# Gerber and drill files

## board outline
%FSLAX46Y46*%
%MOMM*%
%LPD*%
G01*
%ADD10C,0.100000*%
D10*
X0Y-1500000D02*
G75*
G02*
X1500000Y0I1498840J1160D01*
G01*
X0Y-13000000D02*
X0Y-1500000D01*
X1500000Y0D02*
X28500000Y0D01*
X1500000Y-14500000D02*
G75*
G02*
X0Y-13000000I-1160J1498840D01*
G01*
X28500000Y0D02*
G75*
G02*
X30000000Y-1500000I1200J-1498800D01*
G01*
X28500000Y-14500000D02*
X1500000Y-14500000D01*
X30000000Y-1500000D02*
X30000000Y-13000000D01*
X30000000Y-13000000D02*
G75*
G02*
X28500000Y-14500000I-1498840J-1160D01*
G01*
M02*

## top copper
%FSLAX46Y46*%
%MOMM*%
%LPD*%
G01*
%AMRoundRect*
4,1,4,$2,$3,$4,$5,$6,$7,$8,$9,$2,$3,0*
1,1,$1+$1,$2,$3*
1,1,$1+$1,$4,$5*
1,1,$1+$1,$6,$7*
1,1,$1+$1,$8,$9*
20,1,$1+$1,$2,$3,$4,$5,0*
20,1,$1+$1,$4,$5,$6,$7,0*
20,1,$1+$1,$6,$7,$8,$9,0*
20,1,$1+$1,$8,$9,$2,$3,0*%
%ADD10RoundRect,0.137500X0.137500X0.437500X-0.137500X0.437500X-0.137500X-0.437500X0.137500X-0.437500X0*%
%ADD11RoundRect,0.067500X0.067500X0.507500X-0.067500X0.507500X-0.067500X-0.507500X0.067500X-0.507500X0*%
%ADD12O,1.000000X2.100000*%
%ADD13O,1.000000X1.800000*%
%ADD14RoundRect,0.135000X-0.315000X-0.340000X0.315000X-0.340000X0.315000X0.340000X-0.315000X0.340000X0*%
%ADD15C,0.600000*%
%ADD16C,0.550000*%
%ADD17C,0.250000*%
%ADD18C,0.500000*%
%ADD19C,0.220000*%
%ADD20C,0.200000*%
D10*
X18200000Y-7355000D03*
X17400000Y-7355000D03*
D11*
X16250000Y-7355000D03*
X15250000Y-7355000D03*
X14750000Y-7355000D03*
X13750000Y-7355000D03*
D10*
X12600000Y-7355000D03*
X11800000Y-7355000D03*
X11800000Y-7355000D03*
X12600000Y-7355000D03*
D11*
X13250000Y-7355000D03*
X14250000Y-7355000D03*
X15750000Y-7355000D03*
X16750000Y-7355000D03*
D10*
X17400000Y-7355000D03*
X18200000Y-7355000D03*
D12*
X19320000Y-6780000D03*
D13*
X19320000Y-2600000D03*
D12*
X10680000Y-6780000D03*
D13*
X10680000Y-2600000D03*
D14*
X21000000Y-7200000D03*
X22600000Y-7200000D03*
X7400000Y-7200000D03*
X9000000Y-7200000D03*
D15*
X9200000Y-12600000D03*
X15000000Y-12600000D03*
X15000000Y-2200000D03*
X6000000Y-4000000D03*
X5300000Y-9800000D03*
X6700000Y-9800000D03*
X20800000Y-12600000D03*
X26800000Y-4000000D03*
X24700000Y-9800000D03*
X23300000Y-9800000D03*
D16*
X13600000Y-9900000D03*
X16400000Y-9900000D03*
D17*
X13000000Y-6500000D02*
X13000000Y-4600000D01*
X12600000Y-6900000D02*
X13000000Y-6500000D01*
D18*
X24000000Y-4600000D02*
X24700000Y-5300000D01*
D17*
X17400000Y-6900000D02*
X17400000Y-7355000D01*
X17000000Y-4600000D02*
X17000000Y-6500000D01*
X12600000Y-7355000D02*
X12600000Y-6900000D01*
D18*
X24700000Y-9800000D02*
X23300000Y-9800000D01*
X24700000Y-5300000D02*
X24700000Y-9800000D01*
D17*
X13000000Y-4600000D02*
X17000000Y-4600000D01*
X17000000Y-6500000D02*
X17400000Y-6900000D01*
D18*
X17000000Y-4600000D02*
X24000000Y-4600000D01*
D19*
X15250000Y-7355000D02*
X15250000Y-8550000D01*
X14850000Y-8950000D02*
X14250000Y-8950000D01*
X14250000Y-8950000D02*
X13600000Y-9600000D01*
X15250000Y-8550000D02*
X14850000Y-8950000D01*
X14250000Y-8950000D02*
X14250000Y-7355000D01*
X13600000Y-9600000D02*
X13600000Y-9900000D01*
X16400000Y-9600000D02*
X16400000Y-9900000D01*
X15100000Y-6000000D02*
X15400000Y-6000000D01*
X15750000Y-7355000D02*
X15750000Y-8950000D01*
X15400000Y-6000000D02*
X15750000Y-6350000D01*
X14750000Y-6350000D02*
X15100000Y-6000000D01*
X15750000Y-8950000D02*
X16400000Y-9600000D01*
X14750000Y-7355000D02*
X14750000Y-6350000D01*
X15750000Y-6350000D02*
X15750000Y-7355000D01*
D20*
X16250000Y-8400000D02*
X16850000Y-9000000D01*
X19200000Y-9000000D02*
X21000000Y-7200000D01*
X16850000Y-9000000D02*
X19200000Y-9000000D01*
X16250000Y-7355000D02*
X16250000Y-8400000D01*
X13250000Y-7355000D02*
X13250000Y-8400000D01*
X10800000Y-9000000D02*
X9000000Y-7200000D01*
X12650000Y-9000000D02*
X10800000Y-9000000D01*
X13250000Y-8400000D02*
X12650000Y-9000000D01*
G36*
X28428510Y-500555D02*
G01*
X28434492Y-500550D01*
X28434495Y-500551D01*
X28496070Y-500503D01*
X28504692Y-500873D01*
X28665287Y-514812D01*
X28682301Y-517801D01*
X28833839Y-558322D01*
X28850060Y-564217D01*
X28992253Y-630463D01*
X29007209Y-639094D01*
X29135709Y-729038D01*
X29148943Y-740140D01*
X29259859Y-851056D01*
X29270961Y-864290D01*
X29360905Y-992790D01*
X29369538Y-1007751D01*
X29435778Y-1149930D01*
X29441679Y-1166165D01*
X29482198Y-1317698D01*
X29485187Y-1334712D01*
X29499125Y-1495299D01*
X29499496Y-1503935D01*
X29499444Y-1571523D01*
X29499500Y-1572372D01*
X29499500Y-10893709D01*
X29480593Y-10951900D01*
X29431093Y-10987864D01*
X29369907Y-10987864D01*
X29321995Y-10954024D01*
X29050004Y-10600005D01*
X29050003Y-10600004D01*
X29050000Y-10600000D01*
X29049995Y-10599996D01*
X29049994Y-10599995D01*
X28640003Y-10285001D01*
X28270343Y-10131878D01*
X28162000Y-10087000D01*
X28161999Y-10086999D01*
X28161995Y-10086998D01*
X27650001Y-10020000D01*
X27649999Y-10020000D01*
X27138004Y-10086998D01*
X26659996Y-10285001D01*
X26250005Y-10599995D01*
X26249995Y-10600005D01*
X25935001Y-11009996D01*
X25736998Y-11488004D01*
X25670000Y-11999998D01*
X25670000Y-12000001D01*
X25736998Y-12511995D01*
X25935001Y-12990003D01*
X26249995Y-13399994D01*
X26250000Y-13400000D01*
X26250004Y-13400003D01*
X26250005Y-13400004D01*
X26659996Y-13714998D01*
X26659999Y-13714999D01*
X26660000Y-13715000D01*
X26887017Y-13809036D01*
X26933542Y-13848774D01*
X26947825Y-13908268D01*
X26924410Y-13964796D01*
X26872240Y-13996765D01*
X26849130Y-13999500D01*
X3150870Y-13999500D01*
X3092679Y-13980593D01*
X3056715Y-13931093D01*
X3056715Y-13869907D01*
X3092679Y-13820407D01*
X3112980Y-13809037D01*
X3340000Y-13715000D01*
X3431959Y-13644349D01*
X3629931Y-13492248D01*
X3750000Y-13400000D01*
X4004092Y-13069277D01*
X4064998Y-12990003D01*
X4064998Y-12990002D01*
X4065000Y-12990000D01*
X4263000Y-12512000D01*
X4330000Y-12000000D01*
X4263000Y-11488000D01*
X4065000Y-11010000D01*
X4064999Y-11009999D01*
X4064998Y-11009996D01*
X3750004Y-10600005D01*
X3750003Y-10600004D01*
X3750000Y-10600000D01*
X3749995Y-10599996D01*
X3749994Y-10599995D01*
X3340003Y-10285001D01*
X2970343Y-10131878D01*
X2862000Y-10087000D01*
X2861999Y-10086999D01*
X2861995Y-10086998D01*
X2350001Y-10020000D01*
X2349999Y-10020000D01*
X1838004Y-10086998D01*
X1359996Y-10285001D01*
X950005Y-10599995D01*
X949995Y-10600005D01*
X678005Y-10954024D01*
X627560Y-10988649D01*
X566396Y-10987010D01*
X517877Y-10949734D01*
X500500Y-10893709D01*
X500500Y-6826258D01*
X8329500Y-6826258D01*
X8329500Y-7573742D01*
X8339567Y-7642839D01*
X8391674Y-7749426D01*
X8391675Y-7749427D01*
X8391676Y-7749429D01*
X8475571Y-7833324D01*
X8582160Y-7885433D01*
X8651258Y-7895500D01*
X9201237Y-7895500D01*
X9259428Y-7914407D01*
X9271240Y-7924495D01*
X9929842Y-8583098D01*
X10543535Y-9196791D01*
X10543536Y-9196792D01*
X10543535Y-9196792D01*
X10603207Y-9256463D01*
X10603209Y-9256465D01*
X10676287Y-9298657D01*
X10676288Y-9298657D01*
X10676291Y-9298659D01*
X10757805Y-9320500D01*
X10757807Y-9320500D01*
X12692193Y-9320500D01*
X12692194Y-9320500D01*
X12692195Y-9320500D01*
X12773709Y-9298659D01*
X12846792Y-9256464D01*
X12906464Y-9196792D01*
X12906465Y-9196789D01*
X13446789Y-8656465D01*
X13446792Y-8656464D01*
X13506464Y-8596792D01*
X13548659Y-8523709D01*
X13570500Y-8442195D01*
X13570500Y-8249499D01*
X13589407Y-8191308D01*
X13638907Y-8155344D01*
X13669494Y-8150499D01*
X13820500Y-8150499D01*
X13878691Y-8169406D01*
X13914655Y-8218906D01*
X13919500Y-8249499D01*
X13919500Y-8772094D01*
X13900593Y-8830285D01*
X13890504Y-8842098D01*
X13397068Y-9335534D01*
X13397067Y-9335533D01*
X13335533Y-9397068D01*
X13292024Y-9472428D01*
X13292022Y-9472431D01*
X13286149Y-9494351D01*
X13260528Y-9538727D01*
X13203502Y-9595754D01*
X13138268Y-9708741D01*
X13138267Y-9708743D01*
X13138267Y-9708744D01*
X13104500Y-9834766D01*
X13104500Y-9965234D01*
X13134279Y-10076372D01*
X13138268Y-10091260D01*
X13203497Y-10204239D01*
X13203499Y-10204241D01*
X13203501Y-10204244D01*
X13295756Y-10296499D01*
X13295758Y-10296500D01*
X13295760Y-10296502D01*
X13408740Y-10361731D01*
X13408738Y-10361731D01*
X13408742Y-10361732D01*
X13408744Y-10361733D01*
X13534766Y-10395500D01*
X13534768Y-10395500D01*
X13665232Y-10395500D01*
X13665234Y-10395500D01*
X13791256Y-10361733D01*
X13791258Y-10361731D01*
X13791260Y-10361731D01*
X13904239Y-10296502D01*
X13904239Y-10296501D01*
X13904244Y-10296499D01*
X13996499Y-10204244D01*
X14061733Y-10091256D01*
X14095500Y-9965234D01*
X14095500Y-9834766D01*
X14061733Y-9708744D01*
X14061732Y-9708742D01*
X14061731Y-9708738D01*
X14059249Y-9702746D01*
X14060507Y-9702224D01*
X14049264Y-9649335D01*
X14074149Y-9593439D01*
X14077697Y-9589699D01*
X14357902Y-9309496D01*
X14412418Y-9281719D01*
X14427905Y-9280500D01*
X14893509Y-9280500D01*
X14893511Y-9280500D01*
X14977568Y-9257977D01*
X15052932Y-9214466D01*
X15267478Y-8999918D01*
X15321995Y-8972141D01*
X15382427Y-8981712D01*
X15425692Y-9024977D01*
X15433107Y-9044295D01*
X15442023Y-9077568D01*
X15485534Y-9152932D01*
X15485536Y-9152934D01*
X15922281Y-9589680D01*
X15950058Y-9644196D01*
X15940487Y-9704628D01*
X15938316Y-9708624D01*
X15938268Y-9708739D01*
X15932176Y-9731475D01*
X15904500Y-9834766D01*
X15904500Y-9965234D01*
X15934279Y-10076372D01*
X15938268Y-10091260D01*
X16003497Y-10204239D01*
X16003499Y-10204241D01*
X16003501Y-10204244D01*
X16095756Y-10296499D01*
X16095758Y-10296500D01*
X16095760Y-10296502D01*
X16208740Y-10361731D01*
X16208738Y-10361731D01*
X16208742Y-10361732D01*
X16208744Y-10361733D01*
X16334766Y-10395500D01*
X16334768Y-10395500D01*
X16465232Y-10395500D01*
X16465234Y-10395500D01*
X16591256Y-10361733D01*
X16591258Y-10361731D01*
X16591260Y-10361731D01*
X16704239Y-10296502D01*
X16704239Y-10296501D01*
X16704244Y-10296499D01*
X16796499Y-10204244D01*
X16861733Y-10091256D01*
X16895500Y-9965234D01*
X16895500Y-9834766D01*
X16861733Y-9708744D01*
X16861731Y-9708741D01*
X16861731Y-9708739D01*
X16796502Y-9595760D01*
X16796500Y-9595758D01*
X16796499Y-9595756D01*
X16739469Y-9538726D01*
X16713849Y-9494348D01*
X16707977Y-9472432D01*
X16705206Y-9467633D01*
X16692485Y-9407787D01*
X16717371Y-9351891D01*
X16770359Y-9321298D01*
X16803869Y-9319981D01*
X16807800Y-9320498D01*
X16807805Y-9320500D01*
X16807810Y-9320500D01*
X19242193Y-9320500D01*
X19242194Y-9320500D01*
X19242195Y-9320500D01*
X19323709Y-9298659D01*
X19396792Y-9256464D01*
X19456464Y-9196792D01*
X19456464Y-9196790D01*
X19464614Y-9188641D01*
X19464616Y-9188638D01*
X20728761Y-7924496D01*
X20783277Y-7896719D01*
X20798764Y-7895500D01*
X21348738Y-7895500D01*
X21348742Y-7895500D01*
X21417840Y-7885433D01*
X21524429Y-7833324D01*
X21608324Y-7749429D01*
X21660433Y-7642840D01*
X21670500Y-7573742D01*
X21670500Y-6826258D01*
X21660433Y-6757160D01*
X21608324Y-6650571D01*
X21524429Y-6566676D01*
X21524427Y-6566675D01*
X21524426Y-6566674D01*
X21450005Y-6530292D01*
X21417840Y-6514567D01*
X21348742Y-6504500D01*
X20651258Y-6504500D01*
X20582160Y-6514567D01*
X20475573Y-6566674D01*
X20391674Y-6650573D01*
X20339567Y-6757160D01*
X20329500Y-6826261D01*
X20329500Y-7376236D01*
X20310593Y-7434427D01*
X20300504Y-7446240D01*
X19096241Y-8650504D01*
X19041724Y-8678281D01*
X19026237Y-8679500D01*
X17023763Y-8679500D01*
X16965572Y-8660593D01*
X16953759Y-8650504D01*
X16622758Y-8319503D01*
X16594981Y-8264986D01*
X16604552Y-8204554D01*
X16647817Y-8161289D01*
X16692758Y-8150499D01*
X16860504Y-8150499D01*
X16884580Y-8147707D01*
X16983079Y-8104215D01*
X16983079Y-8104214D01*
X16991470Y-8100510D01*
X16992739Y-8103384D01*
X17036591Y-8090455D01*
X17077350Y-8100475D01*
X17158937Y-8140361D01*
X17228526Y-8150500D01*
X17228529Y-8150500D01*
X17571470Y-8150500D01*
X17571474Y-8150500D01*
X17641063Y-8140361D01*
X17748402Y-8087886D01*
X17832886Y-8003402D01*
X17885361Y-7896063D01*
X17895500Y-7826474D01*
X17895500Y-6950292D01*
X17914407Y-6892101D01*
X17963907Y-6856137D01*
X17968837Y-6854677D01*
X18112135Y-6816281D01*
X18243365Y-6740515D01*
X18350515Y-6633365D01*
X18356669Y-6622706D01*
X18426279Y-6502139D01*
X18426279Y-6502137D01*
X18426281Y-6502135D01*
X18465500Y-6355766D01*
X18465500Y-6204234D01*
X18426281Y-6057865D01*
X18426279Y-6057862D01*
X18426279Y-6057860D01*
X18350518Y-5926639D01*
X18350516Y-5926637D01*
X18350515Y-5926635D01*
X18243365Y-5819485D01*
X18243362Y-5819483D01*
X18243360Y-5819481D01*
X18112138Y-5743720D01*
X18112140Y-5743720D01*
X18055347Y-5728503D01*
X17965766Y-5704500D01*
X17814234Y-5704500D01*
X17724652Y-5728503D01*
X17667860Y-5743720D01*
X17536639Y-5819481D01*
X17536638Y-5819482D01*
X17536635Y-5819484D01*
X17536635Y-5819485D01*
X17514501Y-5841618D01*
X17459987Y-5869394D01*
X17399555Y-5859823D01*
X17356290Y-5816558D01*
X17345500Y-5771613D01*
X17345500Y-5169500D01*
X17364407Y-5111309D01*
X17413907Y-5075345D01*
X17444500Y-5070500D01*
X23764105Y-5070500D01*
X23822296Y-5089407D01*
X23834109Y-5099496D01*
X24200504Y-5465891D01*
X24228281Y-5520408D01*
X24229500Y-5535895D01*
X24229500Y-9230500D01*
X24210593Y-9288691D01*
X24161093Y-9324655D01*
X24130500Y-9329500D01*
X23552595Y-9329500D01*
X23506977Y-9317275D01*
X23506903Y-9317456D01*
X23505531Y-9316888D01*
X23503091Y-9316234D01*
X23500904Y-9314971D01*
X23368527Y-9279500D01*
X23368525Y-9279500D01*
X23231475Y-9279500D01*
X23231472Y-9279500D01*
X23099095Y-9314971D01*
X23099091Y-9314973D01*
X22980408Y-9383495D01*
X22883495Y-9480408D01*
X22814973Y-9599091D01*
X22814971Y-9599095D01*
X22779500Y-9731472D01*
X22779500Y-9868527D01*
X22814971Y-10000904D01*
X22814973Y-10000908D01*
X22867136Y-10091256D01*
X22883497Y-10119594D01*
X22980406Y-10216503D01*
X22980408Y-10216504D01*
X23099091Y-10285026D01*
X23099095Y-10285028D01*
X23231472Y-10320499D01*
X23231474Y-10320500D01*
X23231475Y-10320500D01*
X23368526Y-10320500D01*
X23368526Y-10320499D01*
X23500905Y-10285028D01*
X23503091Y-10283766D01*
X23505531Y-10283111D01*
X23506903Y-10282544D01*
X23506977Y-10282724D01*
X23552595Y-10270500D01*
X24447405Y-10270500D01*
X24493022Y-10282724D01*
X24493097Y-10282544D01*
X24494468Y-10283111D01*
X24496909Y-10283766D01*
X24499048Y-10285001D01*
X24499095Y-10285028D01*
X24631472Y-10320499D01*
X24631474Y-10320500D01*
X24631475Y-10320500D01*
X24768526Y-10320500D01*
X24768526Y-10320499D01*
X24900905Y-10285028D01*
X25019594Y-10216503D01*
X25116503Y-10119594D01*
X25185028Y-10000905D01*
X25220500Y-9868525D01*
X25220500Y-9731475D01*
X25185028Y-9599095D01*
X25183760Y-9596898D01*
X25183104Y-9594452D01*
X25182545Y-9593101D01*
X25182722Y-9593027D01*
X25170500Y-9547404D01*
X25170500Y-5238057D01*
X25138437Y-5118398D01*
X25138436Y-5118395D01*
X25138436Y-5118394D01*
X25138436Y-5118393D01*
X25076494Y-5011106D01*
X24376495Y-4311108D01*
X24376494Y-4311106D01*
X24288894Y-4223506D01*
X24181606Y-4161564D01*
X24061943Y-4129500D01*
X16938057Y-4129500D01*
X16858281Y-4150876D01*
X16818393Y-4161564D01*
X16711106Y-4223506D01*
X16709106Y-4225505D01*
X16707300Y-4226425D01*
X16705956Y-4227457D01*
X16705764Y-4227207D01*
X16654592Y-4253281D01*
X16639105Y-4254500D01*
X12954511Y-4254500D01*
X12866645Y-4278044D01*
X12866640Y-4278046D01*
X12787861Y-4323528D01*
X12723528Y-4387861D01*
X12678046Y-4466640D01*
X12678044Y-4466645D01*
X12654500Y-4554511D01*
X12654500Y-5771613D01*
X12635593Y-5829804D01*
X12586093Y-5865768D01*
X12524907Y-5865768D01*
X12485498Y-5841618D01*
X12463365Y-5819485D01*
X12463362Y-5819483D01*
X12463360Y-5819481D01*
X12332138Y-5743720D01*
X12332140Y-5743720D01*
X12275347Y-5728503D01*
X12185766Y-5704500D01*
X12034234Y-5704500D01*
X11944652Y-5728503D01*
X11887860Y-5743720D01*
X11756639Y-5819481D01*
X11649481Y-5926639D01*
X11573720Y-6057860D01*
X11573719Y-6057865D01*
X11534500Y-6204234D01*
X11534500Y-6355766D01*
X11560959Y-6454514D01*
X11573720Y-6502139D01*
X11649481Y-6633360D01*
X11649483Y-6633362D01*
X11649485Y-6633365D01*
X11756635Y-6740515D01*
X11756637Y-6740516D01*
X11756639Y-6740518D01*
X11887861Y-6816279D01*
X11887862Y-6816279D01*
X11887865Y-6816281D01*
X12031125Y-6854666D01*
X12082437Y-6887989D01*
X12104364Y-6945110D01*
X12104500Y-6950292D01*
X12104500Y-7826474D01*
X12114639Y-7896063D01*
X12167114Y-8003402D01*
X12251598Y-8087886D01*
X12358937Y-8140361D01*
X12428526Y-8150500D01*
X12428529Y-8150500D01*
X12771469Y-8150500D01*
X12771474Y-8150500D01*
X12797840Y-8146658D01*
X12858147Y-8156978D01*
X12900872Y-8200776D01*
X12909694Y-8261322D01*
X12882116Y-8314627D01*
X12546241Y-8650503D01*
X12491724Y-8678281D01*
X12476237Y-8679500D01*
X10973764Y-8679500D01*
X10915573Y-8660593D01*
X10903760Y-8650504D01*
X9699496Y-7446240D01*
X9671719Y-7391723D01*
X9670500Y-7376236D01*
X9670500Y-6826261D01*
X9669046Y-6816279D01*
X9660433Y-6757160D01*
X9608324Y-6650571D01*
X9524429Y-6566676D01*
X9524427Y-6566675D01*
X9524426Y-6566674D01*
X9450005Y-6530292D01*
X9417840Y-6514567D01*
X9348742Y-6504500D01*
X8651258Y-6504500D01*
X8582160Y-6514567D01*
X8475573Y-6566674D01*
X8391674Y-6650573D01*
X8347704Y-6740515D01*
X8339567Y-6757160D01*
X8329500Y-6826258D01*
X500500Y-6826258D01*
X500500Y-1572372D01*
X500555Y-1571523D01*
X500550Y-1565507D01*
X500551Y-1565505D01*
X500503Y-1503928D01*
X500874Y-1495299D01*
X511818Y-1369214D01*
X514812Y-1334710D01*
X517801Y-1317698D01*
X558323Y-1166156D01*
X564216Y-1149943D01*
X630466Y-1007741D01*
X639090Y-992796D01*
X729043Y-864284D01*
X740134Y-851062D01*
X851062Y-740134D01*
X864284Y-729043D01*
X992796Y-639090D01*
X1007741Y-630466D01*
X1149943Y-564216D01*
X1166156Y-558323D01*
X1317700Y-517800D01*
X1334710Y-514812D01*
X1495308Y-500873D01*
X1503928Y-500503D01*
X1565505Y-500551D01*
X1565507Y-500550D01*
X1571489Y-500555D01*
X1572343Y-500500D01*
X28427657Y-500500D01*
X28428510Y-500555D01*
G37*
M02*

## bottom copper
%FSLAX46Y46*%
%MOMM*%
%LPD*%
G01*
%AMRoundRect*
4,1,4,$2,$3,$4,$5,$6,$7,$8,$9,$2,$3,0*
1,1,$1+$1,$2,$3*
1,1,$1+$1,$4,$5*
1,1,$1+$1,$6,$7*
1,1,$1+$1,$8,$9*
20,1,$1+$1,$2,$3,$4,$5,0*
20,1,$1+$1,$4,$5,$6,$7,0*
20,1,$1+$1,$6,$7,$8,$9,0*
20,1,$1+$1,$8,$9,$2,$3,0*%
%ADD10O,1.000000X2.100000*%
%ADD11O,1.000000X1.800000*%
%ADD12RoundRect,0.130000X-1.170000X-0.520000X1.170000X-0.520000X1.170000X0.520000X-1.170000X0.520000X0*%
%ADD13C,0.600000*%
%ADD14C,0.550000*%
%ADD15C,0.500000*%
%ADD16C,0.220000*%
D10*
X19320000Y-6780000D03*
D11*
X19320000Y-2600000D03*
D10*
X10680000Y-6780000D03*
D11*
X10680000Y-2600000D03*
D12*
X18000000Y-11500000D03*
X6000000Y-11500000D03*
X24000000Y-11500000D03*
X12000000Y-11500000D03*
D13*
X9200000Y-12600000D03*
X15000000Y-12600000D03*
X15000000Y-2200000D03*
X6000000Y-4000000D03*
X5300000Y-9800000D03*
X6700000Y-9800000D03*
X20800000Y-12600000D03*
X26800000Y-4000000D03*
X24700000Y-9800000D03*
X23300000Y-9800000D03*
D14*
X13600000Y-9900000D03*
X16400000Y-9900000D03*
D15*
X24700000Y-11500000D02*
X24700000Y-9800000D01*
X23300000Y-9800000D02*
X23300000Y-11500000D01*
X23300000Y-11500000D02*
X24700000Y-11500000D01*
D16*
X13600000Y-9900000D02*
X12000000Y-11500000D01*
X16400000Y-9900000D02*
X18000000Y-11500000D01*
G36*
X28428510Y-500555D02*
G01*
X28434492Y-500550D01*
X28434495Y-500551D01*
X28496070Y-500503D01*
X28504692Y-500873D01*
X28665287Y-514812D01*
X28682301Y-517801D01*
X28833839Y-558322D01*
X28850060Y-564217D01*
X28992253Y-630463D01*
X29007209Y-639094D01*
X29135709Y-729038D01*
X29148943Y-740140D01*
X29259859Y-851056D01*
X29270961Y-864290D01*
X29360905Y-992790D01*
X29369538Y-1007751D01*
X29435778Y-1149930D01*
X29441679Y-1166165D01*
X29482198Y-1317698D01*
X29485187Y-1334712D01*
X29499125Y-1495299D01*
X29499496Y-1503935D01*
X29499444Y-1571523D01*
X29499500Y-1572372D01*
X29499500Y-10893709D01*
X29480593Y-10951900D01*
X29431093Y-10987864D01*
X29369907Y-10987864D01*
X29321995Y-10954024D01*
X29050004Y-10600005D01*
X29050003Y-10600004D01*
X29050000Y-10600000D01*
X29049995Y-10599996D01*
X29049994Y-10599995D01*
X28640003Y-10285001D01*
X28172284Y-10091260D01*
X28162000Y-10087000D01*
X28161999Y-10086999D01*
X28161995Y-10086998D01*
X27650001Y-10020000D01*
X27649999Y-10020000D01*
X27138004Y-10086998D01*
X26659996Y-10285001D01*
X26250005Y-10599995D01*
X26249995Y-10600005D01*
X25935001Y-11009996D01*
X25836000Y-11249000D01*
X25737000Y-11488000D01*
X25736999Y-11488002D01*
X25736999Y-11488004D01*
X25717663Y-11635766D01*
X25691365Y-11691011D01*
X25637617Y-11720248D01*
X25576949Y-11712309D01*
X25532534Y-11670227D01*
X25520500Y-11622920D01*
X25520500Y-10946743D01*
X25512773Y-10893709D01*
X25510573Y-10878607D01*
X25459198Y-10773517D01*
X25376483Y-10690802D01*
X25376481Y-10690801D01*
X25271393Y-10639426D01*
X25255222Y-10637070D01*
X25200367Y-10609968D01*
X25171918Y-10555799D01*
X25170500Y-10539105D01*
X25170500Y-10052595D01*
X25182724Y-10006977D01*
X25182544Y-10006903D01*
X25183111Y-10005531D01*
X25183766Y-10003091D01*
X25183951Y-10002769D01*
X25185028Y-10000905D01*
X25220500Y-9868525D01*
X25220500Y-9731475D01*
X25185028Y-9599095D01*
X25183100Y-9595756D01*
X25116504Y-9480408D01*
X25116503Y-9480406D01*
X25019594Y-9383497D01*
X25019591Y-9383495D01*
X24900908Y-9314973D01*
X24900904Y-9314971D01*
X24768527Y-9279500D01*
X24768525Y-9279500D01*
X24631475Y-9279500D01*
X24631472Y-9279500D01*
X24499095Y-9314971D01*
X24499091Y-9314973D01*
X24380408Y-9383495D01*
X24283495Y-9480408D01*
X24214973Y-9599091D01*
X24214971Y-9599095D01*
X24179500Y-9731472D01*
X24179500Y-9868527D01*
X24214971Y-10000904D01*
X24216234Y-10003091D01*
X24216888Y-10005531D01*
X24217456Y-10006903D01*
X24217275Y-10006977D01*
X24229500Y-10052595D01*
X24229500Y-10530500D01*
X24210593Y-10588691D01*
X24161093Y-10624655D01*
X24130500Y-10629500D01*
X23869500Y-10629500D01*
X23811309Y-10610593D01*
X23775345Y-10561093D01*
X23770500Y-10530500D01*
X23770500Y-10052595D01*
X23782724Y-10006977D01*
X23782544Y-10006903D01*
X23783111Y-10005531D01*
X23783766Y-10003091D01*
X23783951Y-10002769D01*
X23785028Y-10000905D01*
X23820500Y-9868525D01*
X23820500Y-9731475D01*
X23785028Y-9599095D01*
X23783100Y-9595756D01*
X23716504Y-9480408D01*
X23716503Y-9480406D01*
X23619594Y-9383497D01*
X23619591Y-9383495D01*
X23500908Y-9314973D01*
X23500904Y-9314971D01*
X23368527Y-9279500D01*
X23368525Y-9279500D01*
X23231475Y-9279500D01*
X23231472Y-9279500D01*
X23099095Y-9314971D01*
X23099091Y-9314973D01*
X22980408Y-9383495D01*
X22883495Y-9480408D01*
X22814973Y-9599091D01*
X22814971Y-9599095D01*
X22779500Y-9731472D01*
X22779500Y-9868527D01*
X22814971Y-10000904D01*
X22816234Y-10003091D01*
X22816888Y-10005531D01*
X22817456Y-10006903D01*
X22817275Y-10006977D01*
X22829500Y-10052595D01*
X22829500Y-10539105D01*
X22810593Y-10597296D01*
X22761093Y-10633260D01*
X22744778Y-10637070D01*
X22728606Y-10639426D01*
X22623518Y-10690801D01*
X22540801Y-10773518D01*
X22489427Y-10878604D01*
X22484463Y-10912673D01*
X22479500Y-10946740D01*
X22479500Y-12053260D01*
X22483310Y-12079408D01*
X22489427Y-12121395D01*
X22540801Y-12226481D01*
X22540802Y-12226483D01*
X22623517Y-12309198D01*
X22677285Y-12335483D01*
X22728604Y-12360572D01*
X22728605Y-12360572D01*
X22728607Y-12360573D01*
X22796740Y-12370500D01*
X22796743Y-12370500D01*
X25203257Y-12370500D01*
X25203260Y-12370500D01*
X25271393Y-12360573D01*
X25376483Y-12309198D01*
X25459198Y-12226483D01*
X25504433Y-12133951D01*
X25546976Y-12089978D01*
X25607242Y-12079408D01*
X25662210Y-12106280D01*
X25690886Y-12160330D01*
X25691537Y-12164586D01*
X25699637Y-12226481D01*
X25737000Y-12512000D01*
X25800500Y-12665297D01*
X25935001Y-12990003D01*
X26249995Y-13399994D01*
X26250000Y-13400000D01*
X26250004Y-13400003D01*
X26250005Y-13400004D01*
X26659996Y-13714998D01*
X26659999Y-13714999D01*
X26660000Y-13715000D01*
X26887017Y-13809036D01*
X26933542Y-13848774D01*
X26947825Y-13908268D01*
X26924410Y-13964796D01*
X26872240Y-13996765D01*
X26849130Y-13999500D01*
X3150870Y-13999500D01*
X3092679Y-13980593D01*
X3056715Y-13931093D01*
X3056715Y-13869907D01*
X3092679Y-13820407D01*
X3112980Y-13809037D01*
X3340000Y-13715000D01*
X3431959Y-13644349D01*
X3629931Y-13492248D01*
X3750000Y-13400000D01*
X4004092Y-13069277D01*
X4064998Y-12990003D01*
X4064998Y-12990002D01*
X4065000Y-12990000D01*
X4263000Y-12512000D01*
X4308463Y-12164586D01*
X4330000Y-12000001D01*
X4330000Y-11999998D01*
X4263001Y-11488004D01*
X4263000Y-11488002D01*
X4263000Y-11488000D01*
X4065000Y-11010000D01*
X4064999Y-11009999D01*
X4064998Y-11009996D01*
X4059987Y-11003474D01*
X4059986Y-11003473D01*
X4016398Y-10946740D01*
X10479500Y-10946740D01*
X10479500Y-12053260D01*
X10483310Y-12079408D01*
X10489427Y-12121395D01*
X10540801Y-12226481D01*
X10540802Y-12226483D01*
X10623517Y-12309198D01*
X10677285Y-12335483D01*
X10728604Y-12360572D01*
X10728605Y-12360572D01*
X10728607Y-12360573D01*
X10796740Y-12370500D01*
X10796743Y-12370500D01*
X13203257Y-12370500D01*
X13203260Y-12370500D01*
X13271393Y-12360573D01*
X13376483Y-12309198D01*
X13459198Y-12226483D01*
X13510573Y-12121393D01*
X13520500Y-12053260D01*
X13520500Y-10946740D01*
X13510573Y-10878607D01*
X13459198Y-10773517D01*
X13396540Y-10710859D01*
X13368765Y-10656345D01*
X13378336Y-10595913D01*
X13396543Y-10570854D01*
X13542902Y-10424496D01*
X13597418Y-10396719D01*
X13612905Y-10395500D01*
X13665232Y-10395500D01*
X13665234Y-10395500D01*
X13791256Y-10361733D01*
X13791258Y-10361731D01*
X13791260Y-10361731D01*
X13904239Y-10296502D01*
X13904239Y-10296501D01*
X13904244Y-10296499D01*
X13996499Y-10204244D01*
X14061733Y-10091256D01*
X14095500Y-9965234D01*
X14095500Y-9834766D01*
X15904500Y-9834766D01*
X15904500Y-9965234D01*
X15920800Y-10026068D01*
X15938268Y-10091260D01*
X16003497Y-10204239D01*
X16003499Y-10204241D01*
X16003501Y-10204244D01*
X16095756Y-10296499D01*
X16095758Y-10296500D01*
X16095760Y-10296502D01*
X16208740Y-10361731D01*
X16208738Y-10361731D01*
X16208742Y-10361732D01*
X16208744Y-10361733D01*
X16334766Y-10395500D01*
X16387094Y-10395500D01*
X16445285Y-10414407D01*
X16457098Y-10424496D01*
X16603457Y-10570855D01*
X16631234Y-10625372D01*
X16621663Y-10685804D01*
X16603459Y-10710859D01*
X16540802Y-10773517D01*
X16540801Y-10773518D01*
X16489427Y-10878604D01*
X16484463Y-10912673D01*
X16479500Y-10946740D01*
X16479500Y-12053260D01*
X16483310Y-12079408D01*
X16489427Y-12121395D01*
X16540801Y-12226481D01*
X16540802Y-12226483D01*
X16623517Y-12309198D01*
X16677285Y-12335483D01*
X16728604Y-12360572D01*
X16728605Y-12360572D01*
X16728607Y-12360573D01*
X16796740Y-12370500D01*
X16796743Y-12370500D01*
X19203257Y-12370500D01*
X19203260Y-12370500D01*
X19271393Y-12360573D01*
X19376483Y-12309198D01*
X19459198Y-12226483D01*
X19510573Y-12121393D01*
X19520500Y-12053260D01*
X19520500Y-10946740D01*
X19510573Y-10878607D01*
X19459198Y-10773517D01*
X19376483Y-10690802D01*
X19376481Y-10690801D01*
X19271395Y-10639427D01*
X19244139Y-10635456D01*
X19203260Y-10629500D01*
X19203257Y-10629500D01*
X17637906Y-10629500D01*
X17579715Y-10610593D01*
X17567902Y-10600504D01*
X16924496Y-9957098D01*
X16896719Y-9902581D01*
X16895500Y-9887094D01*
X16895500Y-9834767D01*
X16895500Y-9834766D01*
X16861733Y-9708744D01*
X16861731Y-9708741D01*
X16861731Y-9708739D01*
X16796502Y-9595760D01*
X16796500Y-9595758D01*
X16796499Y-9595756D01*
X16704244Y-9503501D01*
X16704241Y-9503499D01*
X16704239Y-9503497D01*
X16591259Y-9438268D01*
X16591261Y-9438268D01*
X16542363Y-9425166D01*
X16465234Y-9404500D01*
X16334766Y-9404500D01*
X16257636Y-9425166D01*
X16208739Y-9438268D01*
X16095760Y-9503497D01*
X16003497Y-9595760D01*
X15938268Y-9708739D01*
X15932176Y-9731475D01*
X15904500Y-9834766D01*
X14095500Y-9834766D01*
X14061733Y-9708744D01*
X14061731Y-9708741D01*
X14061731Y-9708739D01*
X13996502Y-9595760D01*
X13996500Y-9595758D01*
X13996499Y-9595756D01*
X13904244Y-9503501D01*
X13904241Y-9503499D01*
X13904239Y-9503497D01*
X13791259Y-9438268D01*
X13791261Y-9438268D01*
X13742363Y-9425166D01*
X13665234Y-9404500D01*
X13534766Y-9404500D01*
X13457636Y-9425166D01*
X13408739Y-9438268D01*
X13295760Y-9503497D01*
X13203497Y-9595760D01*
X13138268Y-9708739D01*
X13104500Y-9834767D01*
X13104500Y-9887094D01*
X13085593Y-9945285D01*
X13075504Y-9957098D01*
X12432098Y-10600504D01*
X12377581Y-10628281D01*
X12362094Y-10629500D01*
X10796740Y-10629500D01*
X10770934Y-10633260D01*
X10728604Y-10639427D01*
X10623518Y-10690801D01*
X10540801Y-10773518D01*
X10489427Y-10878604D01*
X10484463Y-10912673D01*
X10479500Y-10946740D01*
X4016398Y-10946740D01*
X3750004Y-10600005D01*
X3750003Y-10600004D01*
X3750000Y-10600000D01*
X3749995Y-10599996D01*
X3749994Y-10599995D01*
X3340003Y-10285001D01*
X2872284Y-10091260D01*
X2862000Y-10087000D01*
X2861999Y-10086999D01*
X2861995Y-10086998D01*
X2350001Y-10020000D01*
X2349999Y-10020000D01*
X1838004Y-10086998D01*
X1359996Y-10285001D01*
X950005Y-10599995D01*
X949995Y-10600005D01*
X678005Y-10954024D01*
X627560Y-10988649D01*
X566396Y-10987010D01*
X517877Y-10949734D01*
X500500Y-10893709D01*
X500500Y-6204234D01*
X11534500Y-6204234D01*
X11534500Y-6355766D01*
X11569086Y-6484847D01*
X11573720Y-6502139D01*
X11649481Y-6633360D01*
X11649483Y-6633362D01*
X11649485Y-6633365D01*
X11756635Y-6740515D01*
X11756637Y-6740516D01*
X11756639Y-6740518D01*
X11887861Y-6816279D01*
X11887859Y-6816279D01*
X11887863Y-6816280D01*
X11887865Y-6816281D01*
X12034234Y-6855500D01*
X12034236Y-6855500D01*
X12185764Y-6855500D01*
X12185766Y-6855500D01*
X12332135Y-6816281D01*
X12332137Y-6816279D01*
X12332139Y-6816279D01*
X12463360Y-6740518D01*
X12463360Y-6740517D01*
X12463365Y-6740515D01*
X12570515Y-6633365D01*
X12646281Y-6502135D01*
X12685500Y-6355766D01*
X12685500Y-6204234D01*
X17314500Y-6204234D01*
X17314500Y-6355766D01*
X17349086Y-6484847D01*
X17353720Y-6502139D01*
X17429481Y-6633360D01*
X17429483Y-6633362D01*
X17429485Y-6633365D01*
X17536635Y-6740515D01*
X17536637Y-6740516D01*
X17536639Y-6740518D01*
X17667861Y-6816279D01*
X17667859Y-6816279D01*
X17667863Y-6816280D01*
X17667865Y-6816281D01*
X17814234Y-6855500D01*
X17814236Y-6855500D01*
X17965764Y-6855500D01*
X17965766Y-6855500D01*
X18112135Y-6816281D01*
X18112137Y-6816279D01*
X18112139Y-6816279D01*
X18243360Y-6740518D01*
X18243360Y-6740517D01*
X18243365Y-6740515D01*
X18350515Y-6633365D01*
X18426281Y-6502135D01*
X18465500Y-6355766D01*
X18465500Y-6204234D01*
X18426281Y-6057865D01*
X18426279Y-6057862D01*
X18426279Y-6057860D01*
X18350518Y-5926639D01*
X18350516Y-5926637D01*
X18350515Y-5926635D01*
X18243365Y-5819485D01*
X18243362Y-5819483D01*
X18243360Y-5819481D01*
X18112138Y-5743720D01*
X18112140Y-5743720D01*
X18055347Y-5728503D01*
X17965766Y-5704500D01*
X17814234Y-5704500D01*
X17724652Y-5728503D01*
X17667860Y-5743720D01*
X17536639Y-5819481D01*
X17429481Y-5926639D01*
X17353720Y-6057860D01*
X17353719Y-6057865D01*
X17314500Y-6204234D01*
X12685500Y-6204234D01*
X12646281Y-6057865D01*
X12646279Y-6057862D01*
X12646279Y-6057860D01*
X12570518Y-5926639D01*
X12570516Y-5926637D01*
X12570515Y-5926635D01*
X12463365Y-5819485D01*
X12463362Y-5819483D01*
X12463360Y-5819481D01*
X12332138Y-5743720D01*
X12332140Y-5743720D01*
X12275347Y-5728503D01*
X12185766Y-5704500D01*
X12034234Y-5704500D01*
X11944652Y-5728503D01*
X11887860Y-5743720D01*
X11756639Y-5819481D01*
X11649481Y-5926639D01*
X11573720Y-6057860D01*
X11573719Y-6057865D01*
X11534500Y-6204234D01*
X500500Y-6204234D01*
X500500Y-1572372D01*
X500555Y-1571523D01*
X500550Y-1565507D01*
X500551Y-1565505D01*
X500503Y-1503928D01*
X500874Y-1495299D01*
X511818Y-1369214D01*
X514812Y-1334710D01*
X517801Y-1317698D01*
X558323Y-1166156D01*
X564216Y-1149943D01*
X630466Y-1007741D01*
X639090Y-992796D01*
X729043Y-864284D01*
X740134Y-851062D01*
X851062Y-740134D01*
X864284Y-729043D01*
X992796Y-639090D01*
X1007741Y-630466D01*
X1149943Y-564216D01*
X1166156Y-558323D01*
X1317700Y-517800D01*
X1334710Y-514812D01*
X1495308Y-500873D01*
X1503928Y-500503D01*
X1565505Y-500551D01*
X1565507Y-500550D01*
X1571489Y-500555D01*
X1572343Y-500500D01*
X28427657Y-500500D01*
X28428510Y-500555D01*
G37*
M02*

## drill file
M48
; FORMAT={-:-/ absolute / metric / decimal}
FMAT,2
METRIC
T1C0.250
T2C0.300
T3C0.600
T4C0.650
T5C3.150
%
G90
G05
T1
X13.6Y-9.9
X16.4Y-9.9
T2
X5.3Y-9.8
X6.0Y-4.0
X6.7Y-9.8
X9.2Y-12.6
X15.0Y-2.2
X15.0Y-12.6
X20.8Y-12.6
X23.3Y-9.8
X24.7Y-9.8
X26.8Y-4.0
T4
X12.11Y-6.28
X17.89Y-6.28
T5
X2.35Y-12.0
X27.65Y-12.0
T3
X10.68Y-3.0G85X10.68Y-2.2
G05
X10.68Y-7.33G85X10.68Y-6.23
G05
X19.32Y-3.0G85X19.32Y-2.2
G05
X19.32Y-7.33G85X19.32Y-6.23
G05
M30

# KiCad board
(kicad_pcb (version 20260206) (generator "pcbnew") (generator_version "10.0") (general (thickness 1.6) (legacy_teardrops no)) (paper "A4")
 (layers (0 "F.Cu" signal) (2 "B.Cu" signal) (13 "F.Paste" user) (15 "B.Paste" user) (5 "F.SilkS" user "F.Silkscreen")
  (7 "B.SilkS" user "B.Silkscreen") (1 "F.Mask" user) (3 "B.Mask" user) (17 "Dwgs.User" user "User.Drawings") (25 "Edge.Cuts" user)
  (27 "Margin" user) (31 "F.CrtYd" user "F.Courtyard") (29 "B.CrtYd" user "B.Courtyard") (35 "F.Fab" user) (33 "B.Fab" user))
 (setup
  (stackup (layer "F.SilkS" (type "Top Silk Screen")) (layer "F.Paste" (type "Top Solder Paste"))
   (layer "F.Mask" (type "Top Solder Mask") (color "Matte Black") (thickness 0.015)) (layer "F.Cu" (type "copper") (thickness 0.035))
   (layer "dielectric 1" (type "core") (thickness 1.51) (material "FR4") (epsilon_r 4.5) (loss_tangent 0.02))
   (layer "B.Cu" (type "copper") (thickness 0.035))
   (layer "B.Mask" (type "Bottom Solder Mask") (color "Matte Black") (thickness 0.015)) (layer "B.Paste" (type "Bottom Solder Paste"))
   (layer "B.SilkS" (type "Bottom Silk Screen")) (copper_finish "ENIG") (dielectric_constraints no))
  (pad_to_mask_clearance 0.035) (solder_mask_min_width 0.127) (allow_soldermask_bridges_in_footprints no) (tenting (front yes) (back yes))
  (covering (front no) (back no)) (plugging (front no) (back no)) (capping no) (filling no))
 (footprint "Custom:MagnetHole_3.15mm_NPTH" (layer "F.Cu") (at 27.65 12)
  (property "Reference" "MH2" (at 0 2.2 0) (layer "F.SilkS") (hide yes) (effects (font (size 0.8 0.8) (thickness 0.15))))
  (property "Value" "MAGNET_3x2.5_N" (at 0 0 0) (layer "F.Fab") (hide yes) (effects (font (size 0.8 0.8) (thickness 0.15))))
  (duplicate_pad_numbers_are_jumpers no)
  (pad "" np_thru_hole circle (at 0 0) (size 3.15 3.15) (drill 3.15) (layers "*.Cu" "*.Mask")))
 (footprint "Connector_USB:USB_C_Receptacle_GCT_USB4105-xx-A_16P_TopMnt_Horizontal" (layer "F.Cu") (at 15 3.675 180)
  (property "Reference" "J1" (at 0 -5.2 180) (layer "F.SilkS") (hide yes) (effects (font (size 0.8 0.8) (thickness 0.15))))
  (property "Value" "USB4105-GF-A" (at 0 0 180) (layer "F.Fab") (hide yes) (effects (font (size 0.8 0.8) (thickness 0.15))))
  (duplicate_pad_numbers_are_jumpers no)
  (pad "" np_thru_hole circle (at -2.89 -2.605 180) (size 0.65 0.65) (drill 0.65) (layers "*.Cu" "*.Mask"))
  (pad "" np_thru_hole circle (at 2.89 -2.605 180) (size 0.65 0.65) (drill 0.65) (layers "*.Cu" "*.Mask"))
  (pad "A1" smd roundrect (at -3.2 -3.68 180) (size 0.55 1.15) (layers "F.Cu" "F.Mask" "F.Paste") (roundrect_rratio 0.25) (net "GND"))
  (pad "A4" smd roundrect (at -2.4 -3.68 180) (size 0.55 1.15) (layers "F.Cu" "F.Mask" "F.Paste") (roundrect_rratio 0.25) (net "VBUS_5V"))
  (pad "A5" smd roundrect (at -1.25 -3.68 180) (size 0.27 1.15) (layers "F.Cu" "F.Mask" "F.Paste") (roundrect_rratio 0.25) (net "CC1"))
  (pad "A6" smd roundrect (at -0.25 -3.68 180) (size 0.27 1.15) (layers "F.Cu" "F.Mask" "F.Paste") (roundrect_rratio 0.25) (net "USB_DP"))
  (pad "A7" smd roundrect (at 0.25 -3.68 180) (size 0.27 1.15) (layers "F.Cu" "F.Mask" "F.Paste") (roundrect_rratio 0.25) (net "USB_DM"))
  (pad "A8" smd roundrect (at 1.25 -3.68 180) (size 0.27 1.15) (layers "F.Cu" "F.Mask" "F.Paste") (roundrect_rratio 0.25))
  (pad "A9" smd roundrect (at 2.4 -3.68 180) (size 0.55 1.15) (layers "F.Cu" "F.Mask" "F.Paste") (roundrect_rratio 0.25) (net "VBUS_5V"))
  (pad "A12" smd roundrect (at 3.2 -3.68 180) (size 0.55 1.15) (layers "F.Cu" "F.Mask" "F.Paste") (roundrect_rratio 0.25) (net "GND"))
  (pad "B1" smd roundrect (at 3.2 -3.68 180) (size 0.55 1.15) (layers "F.Cu" "F.Mask" "F.Paste") (roundrect_rratio 0.25) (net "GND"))
  (pad "B4" smd roundrect (at 2.4 -3.68 180) (size 0.55 1.15) (layers "F.Cu" "F.Mask" "F.Paste") (roundrect_rratio 0.25) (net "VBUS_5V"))
  (pad "B5" smd roundrect (at 1.75 -3.68 180) (size 0.27 1.15) (layers "F.Cu" "F.Mask" "F.Paste") (roundrect_rratio 0.25) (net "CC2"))
  (pad "B6" smd roundrect (at 0.75 -3.68 180) (size 0.27 1.15) (layers "F.Cu" "F.Mask" "F.Paste") (roundrect_rratio 0.25) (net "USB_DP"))
  (pad "B7" smd roundrect (at -0.75 -3.68 180) (size 0.27 1.15) (layers "F.Cu" "F.Mask" "F.Paste") (roundrect_rratio 0.25) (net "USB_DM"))
  (pad "B8" smd roundrect (at -1.75 -3.68 180) (size 0.27 1.15) (layers "F.Cu" "F.Mask" "F.Paste") (roundrect_rratio 0.25))
  (pad "B9" smd roundrect (at -2.4 -3.68 180) (size 0.55 1.15) (layers "F.Cu" "F.Mask" "F.Paste") (roundrect_rratio 0.25) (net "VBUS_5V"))
  (pad "B12" smd roundrect (at -3.2 -3.68 180) (size 0.55 1.15) (layers "F.Cu" "F.Mask" "F.Paste") (roundrect_rratio 0.25) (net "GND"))
  (pad "SH1" thru_hole oval (at -4.32 -3.105 180) (size 1 2.1) (drill oval 0.6 1.7) (layers "*.Cu" "*.Mask" "F.Paste")
   (remove_unused_layers no) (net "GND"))
  (pad "SH2" thru_hole oval (at -4.32 1.075 180) (size 1 1.8) (drill oval 0.6 1.4) (layers "*.Cu" "*.Mask" "F.Paste")
   (remove_unused_layers no) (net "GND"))
  (pad "SH3" thru_hole oval (at 4.32 -3.105 180) (size 1 2.1) (drill oval 0.6 1.7) (layers "*.Cu" "*.Mask" "F.Paste")
   (remove_unused_layers no) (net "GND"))
  (pad "SH4" thru_hole oval (at 4.32 1.075 180) (size 1 1.8) (drill oval 0.6 1.4) (layers "*.Cu" "*.Mask" "F.Paste")
   (remove_unused_layers no) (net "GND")))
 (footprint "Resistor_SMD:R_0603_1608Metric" (layer "F.Cu") (at 21.8 7.2)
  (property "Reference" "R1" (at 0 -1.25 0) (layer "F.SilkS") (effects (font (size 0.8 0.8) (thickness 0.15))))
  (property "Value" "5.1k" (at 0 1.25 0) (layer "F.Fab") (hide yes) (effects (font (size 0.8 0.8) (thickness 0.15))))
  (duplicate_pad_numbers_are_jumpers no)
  (pad "1" smd roundrect (at -0.8 0) (size 0.9 0.95) (layers "F.Cu" "F.Mask" "F.Paste") (roundrect_rratio 0.15) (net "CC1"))
  (pad "2" smd roundrect (at 0.8 0) (size 0.9 0.95) (layers "F.Cu" "F.Mask" "F.Paste") (roundrect_rratio 0.15) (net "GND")))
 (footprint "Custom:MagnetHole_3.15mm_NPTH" (layer "F.Cu") (at 2.35 12)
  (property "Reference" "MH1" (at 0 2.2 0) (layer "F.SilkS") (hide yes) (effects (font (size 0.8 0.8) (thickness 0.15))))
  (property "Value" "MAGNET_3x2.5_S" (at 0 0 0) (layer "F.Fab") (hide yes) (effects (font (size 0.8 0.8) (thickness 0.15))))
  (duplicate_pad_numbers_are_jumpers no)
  (pad "" np_thru_hole circle (at 0 0) (size 3.15 3.15) (drill 3.15) (layers "*.Cu" "*.Mask")))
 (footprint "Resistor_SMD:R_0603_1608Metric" (layer "F.Cu") (at 8.2 7.2)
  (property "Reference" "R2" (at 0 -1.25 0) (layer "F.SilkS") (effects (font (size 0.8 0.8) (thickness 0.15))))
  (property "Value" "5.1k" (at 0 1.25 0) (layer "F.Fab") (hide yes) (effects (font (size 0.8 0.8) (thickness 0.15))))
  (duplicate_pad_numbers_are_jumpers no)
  (pad "1" smd roundrect (at -0.8 0) (size 0.9 0.95) (layers "F.Cu" "F.Mask" "F.Paste") (roundrect_rratio 0.15) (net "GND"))
  (pad "2" smd roundrect (at 0.8 0) (size 0.9 0.95) (layers "F.Cu" "F.Mask" "F.Paste") (roundrect_rratio 0.15) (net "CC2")))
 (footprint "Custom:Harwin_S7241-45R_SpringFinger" (layer "B.Cu") (at 18 11.5)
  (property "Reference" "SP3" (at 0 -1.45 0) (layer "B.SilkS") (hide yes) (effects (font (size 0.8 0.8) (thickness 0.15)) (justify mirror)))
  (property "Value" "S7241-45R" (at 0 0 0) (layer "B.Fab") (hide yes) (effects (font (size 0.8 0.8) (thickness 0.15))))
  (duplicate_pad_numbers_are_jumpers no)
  (pad "1" smd roundrect (at 0 0) (size 2.6 1.3) (layers "B.Cu" "B.Mask" "B.Paste") (roundrect_rratio 0.1) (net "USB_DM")))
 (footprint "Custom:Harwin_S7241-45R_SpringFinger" (layer "B.Cu") (at 6 11.5)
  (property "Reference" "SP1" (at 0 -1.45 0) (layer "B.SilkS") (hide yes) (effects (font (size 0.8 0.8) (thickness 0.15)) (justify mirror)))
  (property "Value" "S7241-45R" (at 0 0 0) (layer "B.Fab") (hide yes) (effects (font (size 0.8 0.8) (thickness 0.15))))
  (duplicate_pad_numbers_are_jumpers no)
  (pad "1" smd roundrect (at 0 0) (size 2.6 1.3) (layers "B.Cu" "B.Mask" "B.Paste") (roundrect_rratio 0.1) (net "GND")))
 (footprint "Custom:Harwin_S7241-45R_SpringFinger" (layer "B.Cu") (at 24 11.5)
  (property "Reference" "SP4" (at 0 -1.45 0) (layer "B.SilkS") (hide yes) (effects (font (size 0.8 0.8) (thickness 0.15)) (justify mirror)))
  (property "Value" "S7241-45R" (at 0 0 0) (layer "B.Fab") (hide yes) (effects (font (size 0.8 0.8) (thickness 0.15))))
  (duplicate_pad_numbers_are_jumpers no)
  (pad "1" smd roundrect (at 0 0) (size 2.6 1.3) (layers "B.Cu" "B.Mask" "B.Paste") (roundrect_rratio 0.1) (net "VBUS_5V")))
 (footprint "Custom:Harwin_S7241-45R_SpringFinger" (layer "B.Cu") (at 12 11.5)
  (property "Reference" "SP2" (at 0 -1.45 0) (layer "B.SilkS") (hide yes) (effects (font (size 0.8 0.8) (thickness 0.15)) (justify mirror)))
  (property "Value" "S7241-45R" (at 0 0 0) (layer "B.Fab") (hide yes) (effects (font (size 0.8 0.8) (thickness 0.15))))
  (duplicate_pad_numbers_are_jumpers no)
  (pad "1" smd roundrect (at 0 0) (size 2.6 1.3) (layers "B.Cu" "B.Mask" "B.Paste") (roundrect_rratio 0.1) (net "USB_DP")))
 (gr_arc (start 0 1.5) (mid 0.439 0.439) (end 1.5 0) (stroke (width 0.1) (type solid)) (layer "Edge.Cuts"))
 (gr_line (start 0 13) (end 0 1.5) (stroke (width 0.1) (type solid)) (layer "Edge.Cuts"))
 (gr_line (start 1.5 0) (end 28.5 0) (stroke (width 0.1) (type solid)) (layer "Edge.Cuts"))
 (gr_arc (start 1.5 14.5) (mid 0.439 14.061) (end 0 13) (stroke (width 0.1) (type solid)) (layer "Edge.Cuts"))
 (gr_arc (start 28.5 0) (mid 29.561 0.439) (end 30 1.5) (stroke (width 0.1) (type solid)) (layer "Edge.Cuts"))
 (gr_line (start 28.5 14.5) (end 1.5 14.5) (stroke (width 0.1) (type solid)) (layer "Edge.Cuts"))
 (gr_line (start 30 1.5) (end 30 13) (stroke (width 0.1) (type solid)) (layer "Edge.Cuts"))
 (gr_arc (start 30 13) (mid 29.561 14.061) (end 28.5 14.5) (stroke (width 0.1) (type solid)) (layer "Edge.Cuts"))
 (via (at 9.2 12.6) (size 0.6) (drill 0.3) (layers "F.Cu" "B.Cu") (capping no) (covering (front no) (back no))
  (plugging (front no) (back no)) (filling no) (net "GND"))
 (via (at 15 12.6) (size 0.6) (drill 0.3) (layers "F.Cu" "B.Cu") (capping no) (covering (front no) (back no))
  (plugging (front no) (back no)) (filling no) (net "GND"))
 (via (at 15 2.2) (size 0.6) (drill 0.3) (layers "F.Cu" "B.Cu") (capping no) (covering (front no) (back no)) (plugging (front no) (back no))
  (filling no) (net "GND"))
 (via (at 6 4) (size 0.6) (drill 0.3) (layers "F.Cu" "B.Cu") (capping no) (covering (front no) (back no)) (plugging (front no) (back no))
  (filling no) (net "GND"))
 (via (at 5.3 9.8) (size 0.6) (drill 0.3) (layers "F.Cu" "B.Cu") (capping no) (covering (front no) (back no))
  (plugging (front no) (back no)) (filling no) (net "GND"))
 (via (at 6.7 9.8) (size 0.6) (drill 0.3) (layers "F.Cu" "B.Cu") (capping no) (covering (front no) (back no))
  (plugging (front no) (back no)) (filling no) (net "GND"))
 (via (at 20.8 12.6) (size 0.6) (drill 0.3) (layers "F.Cu" "B.Cu") (capping no) (covering (front no) (back no))
  (plugging (front no) (back no)) (filling no) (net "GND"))
 (via (at 26.8 4) (size 0.6) (drill 0.3) (layers "F.Cu" "B.Cu") (capping no) (covering (front no) (back no)) (plugging (front no) (back no))
  (filling no) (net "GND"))
 (segment (start 13 6.5) (end 13 4.6) (width 0.25) (layer "F.Cu") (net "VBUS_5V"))
 (segment (start 12.6 6.9) (end 13 6.5) (width 0.25) (layer "F.Cu") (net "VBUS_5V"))
 (segment (start 24 4.6) (end 24.7 5.3) (width 0.5) (layer "F.Cu") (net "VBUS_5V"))
 (segment (start 17.4 6.9) (end 17.4 7.355) (width 0.25) (layer "F.Cu") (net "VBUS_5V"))
 (segment (start 17 4.6) (end 17 6.5) (width 0.25) (layer "F.Cu") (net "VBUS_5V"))
 (segment (start 12.6 7.355) (end 12.6 6.9) (width 0.25) (layer "F.Cu") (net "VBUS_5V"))
 (segment (start 24.7 9.8) (end 23.3 9.8) (width 0.5) (layer "F.Cu") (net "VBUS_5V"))
 (segment (start 24.7 5.3) (end 24.7 9.8) (width 0.5) (layer "F.Cu") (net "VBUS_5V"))
 (segment (start 13 4.6) (end 17 4.6) (width 0.25) (layer "F.Cu") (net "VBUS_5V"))
 (segment (start 17 6.5) (end 17.4 6.9) (width 0.25) (layer "F.Cu") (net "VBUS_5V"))
 (segment (start 17 4.6) (end 24 4.6) (width 0.5) (layer "F.Cu") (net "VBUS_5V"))
 (via (at 24.7 9.8) (size 0.6) (drill 0.3) (layers "F.Cu" "B.Cu") (capping no) (covering (front no) (back no))
  (plugging (front no) (back no)) (filling no) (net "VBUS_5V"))
 (via (at 23.3 9.8) (size 0.6) (drill 0.3) (layers "F.Cu" "B.Cu") (capping no) (covering (front no) (back no))
  (plugging (front no) (back no)) (filling no) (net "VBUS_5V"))
 (segment (start 24.7 11.5) (end 24.7 9.8) (width 0.5) (layer "B.Cu") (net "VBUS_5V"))
 (segment (start 23.3 9.8) (end 23.3 11.5) (width 0.5) (layer "B.Cu") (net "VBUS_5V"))
 (segment (start 23.3 11.5) (end 24.7 11.5) (width 0.5) (layer "B.Cu") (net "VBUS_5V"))
 (segment (start 15.25 7.355) (end 15.25 8.55) (width 0.22) (layer "F.Cu") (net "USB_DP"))
 (segment (start 14.85 8.95) (end 14.25 8.95) (width 0.22) (layer "F.Cu") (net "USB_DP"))
 (segment (start 14.25 8.95) (end 13.6 9.6) (width 0.22) (layer "F.Cu") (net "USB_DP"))
 (segment (start 15.25 8.55) (end 14.85 8.95) (width 0.22) (layer "F.Cu") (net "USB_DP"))
 (segment (start 14.25 8.95) (end 14.25 7.355) (width 0.22) (layer "F.Cu") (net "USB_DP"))
 (segment (start 13.6 9.6) (end 13.6 9.9) (width 0.22) (layer "F.Cu") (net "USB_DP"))
 (via (at 13.6 9.9) (size 0.55) (drill 0.25) (layers "F.Cu" "B.Cu") (capping no) (covering (front no) (back no))
  (plugging (front no) (back no)) (filling no) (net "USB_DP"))
 (segment (start 13.6 9.9) (end 12 11.5) (width 0.22) (layer "B.Cu") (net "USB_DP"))
 (segment (start 16.4 9.6) (end 16.4 9.9) (width 0.22) (layer "F.Cu") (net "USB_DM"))
 (segment (start 15.1 6) (end 15.4 6) (width 0.22) (layer "F.Cu") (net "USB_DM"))
 (segment (start 15.75 7.355) (end 15.75 8.95) (width 0.22) (layer "F.Cu") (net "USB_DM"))
 (segment (start 15.4 6) (end 15.75 6.35) (width 0.22) (layer "F.Cu") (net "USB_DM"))
 (segment (start 14.75 6.35) (end 15.1 6) (width 0.22) (layer "F.Cu") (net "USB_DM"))
 (segment (start 15.75 8.95) (end 16.4 9.6) (width 0.22) (layer "F.Cu") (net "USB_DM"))
 (segment (start 14.75 7.355) (end 14.75 6.35) (width 0.22) (layer "F.Cu") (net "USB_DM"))
 (segment (start 15.75 6.35) (end 15.75 7.355) (width 0.22) (layer "F.Cu") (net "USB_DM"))
 (via (at 16.4 9.9) (size 0.55) (drill 0.25) (layers "F.Cu" "B.Cu") (capping no) (covering (front no) (back no))
  (plugging (front no) (back no)) (filling no) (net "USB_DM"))
 (segment (start 16.4 9.9) (end 18 11.5) (width 0.22) (layer "B.Cu") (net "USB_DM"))
 (segment (start 16.25 8.4) (end 16.85 9) (width 0.2) (layer "F.Cu") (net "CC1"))
 (segment (start 19.2 9) (end 21 7.2) (width 0.2) (layer "F.Cu") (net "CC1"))
 (segment (start 16.85 9) (end 19.2 9) (width 0.2) (layer "F.Cu") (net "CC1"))
 (segment (start 16.25 7.355) (end 16.25 8.4) (width 0.2) (layer "F.Cu") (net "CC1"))
 (segment (start 13.25 7.355) (end 13.25 8.4) (width 0.2) (layer "F.Cu") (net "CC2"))
 (segment (start 10.8 9) (end 9 7.2) (width 0.2) (layer "F.Cu") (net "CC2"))
 (segment (start 12.65 9) (end 10.8 9) (width 0.2) (layer "F.Cu") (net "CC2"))
 (segment (start 13.25 8.4) (end 12.65 9) (width 0.2) (layer "F.Cu") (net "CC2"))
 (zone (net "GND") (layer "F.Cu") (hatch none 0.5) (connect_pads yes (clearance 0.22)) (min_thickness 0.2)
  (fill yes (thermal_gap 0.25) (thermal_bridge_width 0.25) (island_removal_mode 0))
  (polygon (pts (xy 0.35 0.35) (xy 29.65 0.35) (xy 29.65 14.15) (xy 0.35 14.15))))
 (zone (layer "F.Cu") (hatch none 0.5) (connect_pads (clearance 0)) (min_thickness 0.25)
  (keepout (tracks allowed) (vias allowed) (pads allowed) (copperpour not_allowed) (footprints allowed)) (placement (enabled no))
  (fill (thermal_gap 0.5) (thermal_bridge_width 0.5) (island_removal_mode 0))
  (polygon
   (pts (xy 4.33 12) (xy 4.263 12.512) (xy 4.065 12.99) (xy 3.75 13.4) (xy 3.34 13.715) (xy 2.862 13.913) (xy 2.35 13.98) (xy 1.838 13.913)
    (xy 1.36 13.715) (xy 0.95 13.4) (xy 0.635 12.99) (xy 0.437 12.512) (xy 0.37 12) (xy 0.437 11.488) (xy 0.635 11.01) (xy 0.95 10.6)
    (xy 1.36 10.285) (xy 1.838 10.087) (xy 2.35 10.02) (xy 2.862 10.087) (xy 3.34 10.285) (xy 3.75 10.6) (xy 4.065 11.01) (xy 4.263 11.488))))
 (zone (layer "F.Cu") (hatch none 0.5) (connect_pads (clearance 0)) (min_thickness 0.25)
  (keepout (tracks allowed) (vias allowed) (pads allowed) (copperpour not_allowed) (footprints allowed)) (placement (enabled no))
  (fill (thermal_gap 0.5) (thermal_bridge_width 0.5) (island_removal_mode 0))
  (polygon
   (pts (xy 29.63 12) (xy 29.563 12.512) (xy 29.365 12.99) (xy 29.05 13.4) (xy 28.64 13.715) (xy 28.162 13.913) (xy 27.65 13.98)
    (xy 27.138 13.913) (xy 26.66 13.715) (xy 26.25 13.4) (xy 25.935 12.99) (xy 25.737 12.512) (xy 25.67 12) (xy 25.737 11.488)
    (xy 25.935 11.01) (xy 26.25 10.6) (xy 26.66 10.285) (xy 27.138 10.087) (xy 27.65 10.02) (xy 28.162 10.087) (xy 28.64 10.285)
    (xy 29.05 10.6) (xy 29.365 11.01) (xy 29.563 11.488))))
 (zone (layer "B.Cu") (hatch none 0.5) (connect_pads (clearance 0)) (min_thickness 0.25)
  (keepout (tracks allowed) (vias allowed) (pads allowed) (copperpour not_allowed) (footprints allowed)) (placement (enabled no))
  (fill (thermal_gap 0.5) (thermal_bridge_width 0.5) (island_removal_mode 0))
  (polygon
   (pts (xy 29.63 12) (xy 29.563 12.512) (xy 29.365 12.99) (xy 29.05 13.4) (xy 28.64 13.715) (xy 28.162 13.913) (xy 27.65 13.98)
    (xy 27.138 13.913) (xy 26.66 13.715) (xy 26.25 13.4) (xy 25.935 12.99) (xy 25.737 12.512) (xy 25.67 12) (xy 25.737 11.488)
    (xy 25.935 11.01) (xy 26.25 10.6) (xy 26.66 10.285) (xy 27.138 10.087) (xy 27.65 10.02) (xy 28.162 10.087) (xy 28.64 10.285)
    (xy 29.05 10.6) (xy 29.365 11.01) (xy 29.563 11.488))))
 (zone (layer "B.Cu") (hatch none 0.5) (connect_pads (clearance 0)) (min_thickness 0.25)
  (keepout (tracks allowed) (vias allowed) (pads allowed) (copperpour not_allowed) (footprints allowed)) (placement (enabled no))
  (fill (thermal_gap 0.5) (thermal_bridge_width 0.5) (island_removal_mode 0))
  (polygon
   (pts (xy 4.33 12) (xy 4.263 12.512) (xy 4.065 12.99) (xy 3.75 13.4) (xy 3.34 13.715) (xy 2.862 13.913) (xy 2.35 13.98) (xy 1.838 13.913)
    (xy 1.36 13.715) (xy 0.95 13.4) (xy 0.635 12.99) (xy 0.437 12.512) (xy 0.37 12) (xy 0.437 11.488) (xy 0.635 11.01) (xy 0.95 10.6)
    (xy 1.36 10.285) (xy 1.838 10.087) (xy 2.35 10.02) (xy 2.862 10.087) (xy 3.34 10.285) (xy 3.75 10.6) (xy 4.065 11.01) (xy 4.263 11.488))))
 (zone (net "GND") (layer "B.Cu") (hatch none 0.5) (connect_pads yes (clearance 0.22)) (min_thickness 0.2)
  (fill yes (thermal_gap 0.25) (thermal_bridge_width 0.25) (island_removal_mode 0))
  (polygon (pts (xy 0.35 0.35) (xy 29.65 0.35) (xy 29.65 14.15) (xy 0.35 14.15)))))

